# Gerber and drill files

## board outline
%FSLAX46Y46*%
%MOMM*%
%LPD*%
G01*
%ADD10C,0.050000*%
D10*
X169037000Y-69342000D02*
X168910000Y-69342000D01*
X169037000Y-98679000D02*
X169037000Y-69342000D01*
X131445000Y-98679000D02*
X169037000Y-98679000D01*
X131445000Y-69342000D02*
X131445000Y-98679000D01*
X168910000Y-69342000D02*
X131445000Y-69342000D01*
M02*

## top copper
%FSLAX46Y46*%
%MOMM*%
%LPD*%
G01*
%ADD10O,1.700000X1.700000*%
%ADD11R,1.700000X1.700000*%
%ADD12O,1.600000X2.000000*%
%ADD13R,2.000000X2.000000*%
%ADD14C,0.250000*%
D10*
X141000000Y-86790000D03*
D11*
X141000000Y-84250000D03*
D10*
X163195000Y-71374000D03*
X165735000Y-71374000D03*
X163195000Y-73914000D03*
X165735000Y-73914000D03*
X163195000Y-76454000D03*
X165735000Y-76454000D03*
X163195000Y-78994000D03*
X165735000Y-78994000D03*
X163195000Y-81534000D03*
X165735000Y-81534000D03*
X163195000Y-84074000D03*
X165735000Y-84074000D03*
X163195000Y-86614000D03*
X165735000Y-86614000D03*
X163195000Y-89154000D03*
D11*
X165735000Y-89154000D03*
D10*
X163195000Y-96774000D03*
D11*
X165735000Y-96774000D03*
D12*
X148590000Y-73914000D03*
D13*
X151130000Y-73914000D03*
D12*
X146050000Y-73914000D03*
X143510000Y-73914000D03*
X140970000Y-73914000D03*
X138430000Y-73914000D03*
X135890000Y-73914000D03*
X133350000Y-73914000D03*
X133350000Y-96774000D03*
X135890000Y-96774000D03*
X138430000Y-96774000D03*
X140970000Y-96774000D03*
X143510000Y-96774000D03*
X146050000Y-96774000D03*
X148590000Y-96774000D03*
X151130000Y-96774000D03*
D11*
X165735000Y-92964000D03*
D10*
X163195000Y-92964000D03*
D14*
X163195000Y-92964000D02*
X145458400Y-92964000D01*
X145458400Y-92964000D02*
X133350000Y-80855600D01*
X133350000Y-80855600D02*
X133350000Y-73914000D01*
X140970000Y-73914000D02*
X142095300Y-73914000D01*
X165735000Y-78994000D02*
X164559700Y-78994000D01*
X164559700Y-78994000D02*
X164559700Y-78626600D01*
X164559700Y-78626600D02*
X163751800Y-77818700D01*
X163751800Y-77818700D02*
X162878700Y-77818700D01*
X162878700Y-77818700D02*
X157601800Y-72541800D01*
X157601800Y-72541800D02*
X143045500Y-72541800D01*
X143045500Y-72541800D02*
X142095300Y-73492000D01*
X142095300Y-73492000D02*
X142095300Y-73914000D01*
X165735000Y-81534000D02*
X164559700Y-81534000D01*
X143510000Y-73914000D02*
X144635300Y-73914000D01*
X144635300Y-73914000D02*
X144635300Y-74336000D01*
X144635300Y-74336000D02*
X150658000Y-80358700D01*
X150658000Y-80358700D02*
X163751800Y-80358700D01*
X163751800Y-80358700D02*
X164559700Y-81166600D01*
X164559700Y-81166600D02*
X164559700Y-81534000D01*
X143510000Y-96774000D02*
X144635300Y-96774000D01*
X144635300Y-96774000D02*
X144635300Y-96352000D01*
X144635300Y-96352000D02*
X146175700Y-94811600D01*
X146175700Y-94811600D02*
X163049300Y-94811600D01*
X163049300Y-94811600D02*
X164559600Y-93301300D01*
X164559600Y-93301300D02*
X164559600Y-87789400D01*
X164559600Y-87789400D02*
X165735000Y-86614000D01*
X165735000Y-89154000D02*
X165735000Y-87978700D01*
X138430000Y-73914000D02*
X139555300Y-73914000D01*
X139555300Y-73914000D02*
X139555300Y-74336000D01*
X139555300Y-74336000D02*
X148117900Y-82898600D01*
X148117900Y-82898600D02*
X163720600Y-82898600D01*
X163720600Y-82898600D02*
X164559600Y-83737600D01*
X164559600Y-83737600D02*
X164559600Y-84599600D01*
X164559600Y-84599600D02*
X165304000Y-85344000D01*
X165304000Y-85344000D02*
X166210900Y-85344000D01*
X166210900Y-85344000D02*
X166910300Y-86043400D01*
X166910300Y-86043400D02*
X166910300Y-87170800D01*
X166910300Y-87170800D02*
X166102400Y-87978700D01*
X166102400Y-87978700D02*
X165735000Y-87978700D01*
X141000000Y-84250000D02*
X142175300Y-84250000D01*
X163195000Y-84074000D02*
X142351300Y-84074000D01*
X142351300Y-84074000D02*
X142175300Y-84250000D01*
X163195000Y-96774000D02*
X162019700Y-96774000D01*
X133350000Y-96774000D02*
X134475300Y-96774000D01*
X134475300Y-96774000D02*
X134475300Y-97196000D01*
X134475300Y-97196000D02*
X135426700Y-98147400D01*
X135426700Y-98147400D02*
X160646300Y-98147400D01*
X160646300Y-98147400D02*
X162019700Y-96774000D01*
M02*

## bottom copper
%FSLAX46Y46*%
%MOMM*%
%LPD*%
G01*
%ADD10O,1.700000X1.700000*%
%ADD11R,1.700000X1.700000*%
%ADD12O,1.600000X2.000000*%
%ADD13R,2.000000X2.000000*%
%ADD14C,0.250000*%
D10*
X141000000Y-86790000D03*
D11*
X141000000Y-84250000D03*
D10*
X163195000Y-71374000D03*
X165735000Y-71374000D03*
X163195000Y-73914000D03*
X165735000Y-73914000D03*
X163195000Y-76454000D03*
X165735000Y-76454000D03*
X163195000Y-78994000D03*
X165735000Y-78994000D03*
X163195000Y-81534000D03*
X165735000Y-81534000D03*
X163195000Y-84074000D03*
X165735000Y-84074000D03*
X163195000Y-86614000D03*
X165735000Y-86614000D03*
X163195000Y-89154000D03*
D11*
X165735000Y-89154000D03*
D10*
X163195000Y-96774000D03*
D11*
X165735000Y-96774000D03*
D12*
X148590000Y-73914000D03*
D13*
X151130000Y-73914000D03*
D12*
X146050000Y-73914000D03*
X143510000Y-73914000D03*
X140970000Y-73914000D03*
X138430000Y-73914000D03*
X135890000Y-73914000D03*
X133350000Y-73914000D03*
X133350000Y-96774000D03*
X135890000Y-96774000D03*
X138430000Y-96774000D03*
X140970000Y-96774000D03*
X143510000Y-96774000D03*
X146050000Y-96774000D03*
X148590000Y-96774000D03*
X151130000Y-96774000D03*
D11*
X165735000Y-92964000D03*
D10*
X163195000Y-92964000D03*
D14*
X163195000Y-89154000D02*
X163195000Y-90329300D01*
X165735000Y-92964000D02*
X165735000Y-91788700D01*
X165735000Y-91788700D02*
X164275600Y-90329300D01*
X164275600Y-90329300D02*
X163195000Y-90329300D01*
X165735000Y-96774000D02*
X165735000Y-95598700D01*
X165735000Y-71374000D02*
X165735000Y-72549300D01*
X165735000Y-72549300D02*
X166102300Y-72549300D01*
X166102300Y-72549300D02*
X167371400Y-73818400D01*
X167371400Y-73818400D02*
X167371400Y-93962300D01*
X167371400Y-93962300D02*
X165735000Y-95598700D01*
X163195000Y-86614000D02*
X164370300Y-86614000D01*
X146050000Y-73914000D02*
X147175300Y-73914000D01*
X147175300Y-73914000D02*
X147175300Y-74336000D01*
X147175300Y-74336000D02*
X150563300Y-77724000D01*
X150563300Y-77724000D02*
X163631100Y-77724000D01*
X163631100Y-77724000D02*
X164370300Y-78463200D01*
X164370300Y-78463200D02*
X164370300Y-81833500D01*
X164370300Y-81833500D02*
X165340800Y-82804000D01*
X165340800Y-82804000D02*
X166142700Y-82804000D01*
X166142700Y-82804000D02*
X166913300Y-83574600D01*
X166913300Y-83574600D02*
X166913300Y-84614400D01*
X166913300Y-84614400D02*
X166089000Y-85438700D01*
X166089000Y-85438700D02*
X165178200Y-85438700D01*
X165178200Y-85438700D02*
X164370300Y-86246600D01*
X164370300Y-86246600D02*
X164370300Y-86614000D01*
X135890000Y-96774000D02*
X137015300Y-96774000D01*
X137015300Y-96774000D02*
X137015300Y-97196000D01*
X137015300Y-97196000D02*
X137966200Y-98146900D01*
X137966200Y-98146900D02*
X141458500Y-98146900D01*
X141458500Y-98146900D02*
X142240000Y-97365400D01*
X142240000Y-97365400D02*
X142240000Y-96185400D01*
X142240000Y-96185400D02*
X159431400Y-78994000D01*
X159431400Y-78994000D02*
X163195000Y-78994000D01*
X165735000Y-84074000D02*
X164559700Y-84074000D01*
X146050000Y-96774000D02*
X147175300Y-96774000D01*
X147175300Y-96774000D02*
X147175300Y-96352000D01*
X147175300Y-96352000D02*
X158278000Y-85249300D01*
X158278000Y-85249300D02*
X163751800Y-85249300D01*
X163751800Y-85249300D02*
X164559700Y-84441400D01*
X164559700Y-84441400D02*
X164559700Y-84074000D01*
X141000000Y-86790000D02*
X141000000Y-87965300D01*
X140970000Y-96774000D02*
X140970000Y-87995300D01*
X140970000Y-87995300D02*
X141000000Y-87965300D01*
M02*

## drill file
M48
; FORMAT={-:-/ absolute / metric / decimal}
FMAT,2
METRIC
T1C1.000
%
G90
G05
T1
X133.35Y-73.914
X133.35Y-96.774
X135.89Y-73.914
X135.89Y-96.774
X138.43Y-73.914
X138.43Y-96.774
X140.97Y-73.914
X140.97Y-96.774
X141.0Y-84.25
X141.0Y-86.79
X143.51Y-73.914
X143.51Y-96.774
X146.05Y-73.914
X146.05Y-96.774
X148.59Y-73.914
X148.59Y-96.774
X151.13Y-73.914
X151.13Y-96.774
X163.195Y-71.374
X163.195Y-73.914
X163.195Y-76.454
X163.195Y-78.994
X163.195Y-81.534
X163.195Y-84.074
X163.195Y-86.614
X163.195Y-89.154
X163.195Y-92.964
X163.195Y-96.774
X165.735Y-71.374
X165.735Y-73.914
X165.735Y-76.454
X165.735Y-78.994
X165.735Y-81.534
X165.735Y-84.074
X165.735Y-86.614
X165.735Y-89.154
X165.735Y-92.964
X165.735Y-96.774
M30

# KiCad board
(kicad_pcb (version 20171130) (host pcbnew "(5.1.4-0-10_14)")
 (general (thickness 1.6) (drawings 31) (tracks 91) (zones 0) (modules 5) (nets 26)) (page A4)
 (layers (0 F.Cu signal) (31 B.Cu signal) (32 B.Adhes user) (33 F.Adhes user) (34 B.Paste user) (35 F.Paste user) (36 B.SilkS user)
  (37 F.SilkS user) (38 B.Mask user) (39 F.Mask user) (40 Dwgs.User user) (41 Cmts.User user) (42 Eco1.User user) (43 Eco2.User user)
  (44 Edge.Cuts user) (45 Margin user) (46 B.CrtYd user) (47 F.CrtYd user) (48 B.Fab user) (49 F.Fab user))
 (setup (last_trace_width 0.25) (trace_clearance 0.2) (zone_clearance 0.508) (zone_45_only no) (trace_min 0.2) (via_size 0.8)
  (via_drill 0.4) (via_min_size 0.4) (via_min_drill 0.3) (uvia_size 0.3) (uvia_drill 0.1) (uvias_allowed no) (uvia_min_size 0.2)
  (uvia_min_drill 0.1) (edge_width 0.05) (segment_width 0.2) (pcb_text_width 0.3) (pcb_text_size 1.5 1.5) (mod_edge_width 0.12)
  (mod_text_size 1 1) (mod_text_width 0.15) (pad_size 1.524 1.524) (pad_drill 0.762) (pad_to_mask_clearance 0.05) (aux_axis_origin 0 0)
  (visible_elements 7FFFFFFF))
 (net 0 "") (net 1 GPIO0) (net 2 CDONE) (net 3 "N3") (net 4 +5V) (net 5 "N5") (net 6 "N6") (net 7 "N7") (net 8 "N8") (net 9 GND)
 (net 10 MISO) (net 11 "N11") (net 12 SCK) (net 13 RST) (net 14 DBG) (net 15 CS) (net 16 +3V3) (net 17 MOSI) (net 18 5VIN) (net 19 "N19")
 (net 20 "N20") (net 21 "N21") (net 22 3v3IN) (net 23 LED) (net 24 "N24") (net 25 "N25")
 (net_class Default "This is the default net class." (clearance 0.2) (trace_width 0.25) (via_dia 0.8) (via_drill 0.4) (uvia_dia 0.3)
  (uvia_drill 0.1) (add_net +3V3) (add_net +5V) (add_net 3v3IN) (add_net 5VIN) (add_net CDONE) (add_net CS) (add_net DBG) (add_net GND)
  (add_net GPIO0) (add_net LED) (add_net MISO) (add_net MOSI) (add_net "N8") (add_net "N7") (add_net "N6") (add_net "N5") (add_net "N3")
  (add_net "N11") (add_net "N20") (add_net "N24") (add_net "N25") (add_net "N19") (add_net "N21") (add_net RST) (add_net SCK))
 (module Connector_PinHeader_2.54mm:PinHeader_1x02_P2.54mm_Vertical (layer F.Cu) (at 141 84.25)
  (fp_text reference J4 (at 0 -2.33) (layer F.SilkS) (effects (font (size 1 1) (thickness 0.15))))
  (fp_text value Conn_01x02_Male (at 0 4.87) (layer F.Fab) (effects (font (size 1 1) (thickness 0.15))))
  (pad 2 thru_hole oval (at 0 2.54) (size 1.7 1.7) (drill 1) (layers *.Cu *.Mask) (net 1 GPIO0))
  (pad 1 thru_hole rect (at 0 0) (size 1.7 1.7) (drill 1) (layers *.Cu *.Mask) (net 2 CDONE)))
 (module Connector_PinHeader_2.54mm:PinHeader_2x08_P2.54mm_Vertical (layer F.Cu) (at 165.735 89.154 180)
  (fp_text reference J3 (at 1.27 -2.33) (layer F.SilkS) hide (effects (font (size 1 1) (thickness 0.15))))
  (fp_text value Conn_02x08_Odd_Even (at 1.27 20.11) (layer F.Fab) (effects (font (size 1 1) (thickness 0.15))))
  (pad 16 thru_hole oval (at 2.54 17.78 180) (size 1.7 1.7) (drill 1) (layers *.Cu *.Mask) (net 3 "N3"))
  (pad 15 thru_hole oval (at 0 17.78 180) (size 1.7 1.7) (drill 1) (layers *.Cu *.Mask) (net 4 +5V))
  (pad 14 thru_hole oval (at 2.54 15.24 180) (size 1.7 1.7) (drill 1) (layers *.Cu *.Mask) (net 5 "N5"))
  (pad 13 thru_hole oval (at 0 15.24 180) (size 1.7 1.7) (drill 1) (layers *.Cu *.Mask) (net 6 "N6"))
  (pad 12 thru_hole oval (at 2.54 12.7 180) (size 1.7 1.7) (drill 1) (layers *.Cu *.Mask) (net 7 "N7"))
  (pad 11 thru_hole oval (at 0 12.7 180) (size 1.7 1.7) (drill 1) (layers *.Cu *.Mask) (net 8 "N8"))
  (pad 10 thru_hole oval (at 2.54 10.16 180) (size 1.7 1.7) (drill 1) (layers *.Cu *.Mask) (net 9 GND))
  (pad 9 thru_hole oval (at 0 10.16 180) (size 1.7 1.7) (drill 1) (layers *.Cu *.Mask) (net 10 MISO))
  (pad 8 thru_hole oval (at 2.54 7.62 180) (size 1.7 1.7) (drill 1) (layers *.Cu *.Mask) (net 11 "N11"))
  (pad 7 thru_hole oval (at 0 7.62 180) (size 1.7 1.7) (drill 1) (layers *.Cu *.Mask) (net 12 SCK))
  (pad 6 thru_hole oval (at 2.54 5.08 180) (size 1.7 1.7) (drill 1) (layers *.Cu *.Mask) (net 2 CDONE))
  (pad 5 thru_hole oval (at 0 5.08 180) (size 1.7 1.7) (drill 1) (layers *.Cu *.Mask) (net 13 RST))
  (pad 4 thru_hole oval (at 2.54 2.54 180) (size 1.7 1.7) (drill 1) (layers *.Cu *.Mask) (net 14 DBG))
  (pad 3 thru_hole oval (at 0 2.54 180) (size 1.7 1.7) (drill 1) (layers *.Cu *.Mask) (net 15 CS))
  (pad 2 thru_hole oval (at 2.54 0 180) (size 1.7 1.7) (drill 1) (layers *.Cu *.Mask) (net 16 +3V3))
  (pad 1 thru_hole rect (at 0 0 180) (size 1.7 1.7) (drill 1) (layers *.Cu *.Mask) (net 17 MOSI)))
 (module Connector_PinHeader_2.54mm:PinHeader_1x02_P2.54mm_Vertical (layer F.Cu) (at 165.735 96.774 270)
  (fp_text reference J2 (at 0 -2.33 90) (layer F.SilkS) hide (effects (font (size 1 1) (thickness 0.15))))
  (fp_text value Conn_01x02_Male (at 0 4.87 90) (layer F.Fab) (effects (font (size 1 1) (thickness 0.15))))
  (pad 2 thru_hole oval (at 0 2.54 270) (size 1.7 1.7) (drill 1) (layers *.Cu *.Mask) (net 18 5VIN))
  (pad 1 thru_hole rect (at 0 0 270) (size 1.7 1.7) (drill 1) (layers *.Cu *.Mask) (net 4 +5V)))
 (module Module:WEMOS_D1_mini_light (layer F.Cu) (at 151.13 73.914 270)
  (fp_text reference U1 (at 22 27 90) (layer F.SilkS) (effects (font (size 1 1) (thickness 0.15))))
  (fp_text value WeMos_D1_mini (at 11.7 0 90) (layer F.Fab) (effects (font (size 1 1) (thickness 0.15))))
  (pad 2 thru_hole oval (at 0 2.54 270) (size 2 1.6) (drill 1) (layers *.Cu *.Mask) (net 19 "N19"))
  (pad 1 thru_hole rect (at 0 0 270) (size 2 2) (drill 1) (layers *.Cu *.Mask) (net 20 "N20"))
  (pad 3 thru_hole oval (at 0 5.08 270) (size 2 1.6) (drill 1) (layers *.Cu *.Mask) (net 14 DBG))
  (pad 4 thru_hole oval (at 0 7.62 270) (size 2 1.6) (drill 1) (layers *.Cu *.Mask) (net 12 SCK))
  (pad 5 thru_hole oval (at 0 10.16 270) (size 2 1.6) (drill 1) (layers *.Cu *.Mask) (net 10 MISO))
  (pad 6 thru_hole oval (at 0 12.7 270) (size 2 1.6) (drill 1) (layers *.Cu *.Mask) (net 17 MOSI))
  (pad 7 thru_hole oval (at 0 15.24 270) (size 2 1.6) (drill 1) (layers *.Cu *.Mask) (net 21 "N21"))
  (pad 8 thru_hole oval (at 0 17.78 270) (size 2 1.6) (drill 1) (layers *.Cu *.Mask) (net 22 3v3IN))
  (pad 9 thru_hole oval (at 22.86 17.78 270) (size 2 1.6) (drill 1) (layers *.Cu *.Mask) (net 18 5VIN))
  (pad 10 thru_hole oval (at 22.86 15.24 270) (size 2 1.6) (drill 1) (layers *.Cu *.Mask) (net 9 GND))
  (pad 11 thru_hole oval (at 22.86 12.7 270) (size 2 1.6) (drill 1) (layers *.Cu *.Mask) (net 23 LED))
  (pad 12 thru_hole oval (at 22.86 10.16 270) (size 2 1.6) (drill 1) (layers *.Cu *.Mask) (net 1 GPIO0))
  (pad 13 thru_hole oval (at 22.86 7.62 270) (size 2 1.6) (drill 1) (layers *.Cu *.Mask) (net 15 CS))
  (pad 14 thru_hole oval (at 22.86 5.08 270) (size 2 1.6) (drill 1) (layers *.Cu *.Mask) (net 13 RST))
  (pad 15 thru_hole oval (at 22.86 2.54 270) (size 2 1.6) (drill 1) (layers *.Cu *.Mask) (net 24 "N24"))
  (pad 16 thru_hole oval (at 22.86 0 270) (size 2 1.6) (drill 1) (layers *.Cu *.Mask) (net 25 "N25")))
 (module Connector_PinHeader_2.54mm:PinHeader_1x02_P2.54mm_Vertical (layer F.Cu) (at 165.735 92.964 270)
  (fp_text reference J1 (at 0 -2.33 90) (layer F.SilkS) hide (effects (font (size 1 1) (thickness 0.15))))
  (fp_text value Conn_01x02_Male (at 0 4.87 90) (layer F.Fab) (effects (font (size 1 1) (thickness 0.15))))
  (pad 1 thru_hole rect (at 0 0 270) (size 1.7 1.7) (drill 1) (layers *.Cu *.Mask) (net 16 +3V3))
  (pad 2 thru_hole oval (at 0 2.54 270) (size 1.7 1.7) (drill 1) (layers *.Cu *.Mask) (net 22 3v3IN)))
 (gr_line (start 169.037 69.342) (end 168.91 69.342) (layer Edge.Cuts) (width 0.05))
 (gr_line (start 169.037 98.679) (end 169.037 69.342) (layer Edge.Cuts) (width 0.05))
 (gr_line (start 131.445 98.679) (end 169.037 98.679) (layer Edge.Cuts) (width 0.05))
 (gr_line (start 131.445 69.342) (end 131.445 98.679) (layer Edge.Cuts) (width 0.05))
 (gr_line (start 168.91 69.342) (end 131.445 69.342) (layer Edge.Cuts) (width 0.05))
 (segment (start 163.195 92.964) (end 145.4584 92.964) (width 0.25) (layer F.Cu) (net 22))
 (segment (start 145.4584 92.964) (end 133.35 80.8556) (width 0.25) (layer F.Cu) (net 22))
 (segment (start 133.35 80.8556) (end 133.35 73.914) (width 0.25) (layer F.Cu) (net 22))
 (segment (start 163.195 89.154) (end 163.195 90.3293) (width 0.25) (layer B.Cu) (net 16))
 (segment (start 165.735 92.964) (end 165.735 91.7887) (width 0.25) (layer B.Cu) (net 16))
 (segment (start 165.735 91.7887) (end 164.2756 90.3293) (width 0.25) (layer B.Cu) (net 16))
 (segment (start 164.2756 90.3293) (end 163.195 90.3293) (width 0.25) (layer B.Cu) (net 16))
 (segment (start 165.735 96.774) (end 165.735 95.5987) (width 0.25) (layer B.Cu) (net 4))
 (segment (start 165.735 71.374) (end 165.735 72.5493) (width 0.25) (layer B.Cu) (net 4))
 (segment (start 165.735 72.5493) (end 166.1023 72.5493) (width 0.25) (layer B.Cu) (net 4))
 (segment (start 166.1023 72.5493) (end 167.3714 73.8184) (width 0.25) (layer B.Cu) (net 4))
 (segment (start 167.3714 73.8184) (end 167.3714 93.9623) (width 0.25) (layer B.Cu) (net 4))
 (segment (start 167.3714 93.9623) (end 165.735 95.5987) (width 0.25) (layer B.Cu) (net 4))
 (segment (start 163.195 86.614) (end 164.3703 86.614) (width 0.25) (layer B.Cu) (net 14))
 (segment (start 146.05 73.914) (end 147.1753 73.914) (width 0.25) (layer B.Cu) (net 14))
 (segment (start 147.1753 73.914) (end 147.1753 74.336) (width 0.25) (layer B.Cu) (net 14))
 (segment (start 147.1753 74.336) (end 150.5633 77.724) (width 0.25) (layer B.Cu) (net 14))
 (segment (start 150.5633 77.724) (end 163.6311 77.724) (width 0.25) (layer B.Cu) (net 14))
 (segment (start 163.6311 77.724) (end 164.3703 78.4632) (width 0.25) (layer B.Cu) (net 14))
 (segment (start 164.3703 78.4632) (end 164.3703 81.8335) (width 0.25) (layer B.Cu) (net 14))
 (segment (start 164.3703 81.8335) (end 165.3408 82.804) (width 0.25) (layer B.Cu) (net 14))
 (segment (start 165.3408 82.804) (end 166.1427 82.804) (width 0.25) (layer B.Cu) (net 14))
 (segment (start 166.1427 82.804) (end 166.9133 83.5746) (width 0.25) (layer B.Cu) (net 14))
 (segment (start 166.9133 83.5746) (end 166.9133 84.6144) (width 0.25) (layer B.Cu) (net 14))
 (segment (start 166.9133 84.6144) (end 166.089 85.4387) (width 0.25) (layer B.Cu) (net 14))
 (segment (start 166.089 85.4387) (end 165.1782 85.4387) (width 0.25) (layer B.Cu) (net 14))
 (segment (start 165.1782 85.4387) (end 164.3703 86.2466) (width 0.25) (layer B.Cu) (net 14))
 (segment (start 164.3703 86.2466) (end 164.3703 86.614) (width 0.25) (layer B.Cu) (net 14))
 (segment (start 135.89 96.774) (end 137.0153 96.774) (width 0.25) (layer B.Cu) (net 9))
 (segment (start 137.0153 96.774) (end 137.0153 97.196) (width 0.25) (layer B.Cu) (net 9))
 (segment (start 137.0153 97.196) (end 137.9662 98.1469) (width 0.25) (layer B.Cu) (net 9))
 (segment (start 137.9662 98.1469) (end 141.4585 98.1469) (width 0.25) (layer B.Cu) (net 9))
 (segment (start 141.4585 98.1469) (end 142.24 97.3654) (width 0.25) (layer B.Cu) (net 9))
 (segment (start 142.24 97.3654) (end 142.24 96.1854) (width 0.25) (layer B.Cu) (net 9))
 (segment (start 142.24 96.1854) (end 159.4314 78.994) (width 0.25) (layer B.Cu) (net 9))
 (segment (start 159.4314 78.994) (end 163.195 78.994) (width 0.25) (layer B.Cu) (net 9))
 (segment (start 140.97 73.914) (end 142.0953 73.914) (width 0.25) (layer F.Cu) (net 10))
 (segment (start 165.735 78.994) (end 164.5597 78.994) (width 0.25) (layer F.Cu) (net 10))
 (segment (start 164.5597 78.994) (end 164.5597 78.6266) (width 0.25) (layer F.Cu) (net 10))
 (segment (start 164.5597 78.6266) (end 163.7518 77.8187) (width 0.25) (layer F.Cu) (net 10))
 (segment (start 163.7518 77.8187) (end 162.8787 77.8187) (width 0.25) (layer F.Cu) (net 10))
 (segment (start 162.8787 77.8187) (end 157.6018 72.5418) (width 0.25) (layer F.Cu) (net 10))
 (segment (start 157.6018 72.5418) (end 143.0455 72.5418) (width 0.25) (layer F.Cu) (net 10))
 (segment (start 143.0455 72.5418) (end 142.0953 73.492) (width 0.25) (layer F.Cu) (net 10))
 (segment (start 142.0953 73.492) (end 142.0953 73.914) (width 0.25) (layer F.Cu) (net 10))
 (segment (start 165.735 81.534) (end 164.5597 81.534) (width 0.25) (layer F.Cu) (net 12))
 (segment (start 143.51 73.914) (end 144.6353 73.914) (width 0.25) (layer F.Cu) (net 12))
 (segment (start 144.6353 73.914) (end 144.6353 74.336) (width 0.25) (layer F.Cu) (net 12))
 (segment (start 144.6353 74.336) (end 150.658 80.3587) (width 0.25) (layer F.Cu) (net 12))
 (segment (start 150.658 80.3587) (end 163.7518 80.3587) (width 0.25) (layer F.Cu) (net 12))
 (segment (start 163.7518 80.3587) (end 164.5597 81.1666) (width 0.25) (layer F.Cu) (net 12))
 (segment (start 164.5597 81.1666) (end 164.5597 81.534) (width 0.25) (layer F.Cu) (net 12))
 (segment (start 165.735 84.074) (end 164.5597 84.074) (width 0.25) (layer B.Cu) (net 13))
 (segment (start 146.05 96.774) (end 147.1753 96.774) (width 0.25) (layer B.Cu) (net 13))
 (segment (start 147.1753 96.774) (end 147.1753 96.352) (width 0.25) (layer B.Cu) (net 13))
 (segment (start 147.1753 96.352) (end 158.278 85.2493) (width 0.25) (layer B.Cu) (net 13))
 (segment (start 158.278 85.2493) (end 163.7518 85.2493) (width 0.25) (layer B.Cu) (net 13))
 (segment (start 163.7518 85.2493) (end 164.5597 84.4414) (width 0.25) (layer B.Cu) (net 13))
 (segment (start 164.5597 84.4414) (end 164.5597 84.074) (width 0.25) (layer B.Cu) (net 13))
 (segment (start 143.51 96.774) (end 144.6353 96.774) (width 0.25) (layer F.Cu) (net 15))
 (segment (start 144.6353 96.774) (end 144.6353 96.352) (width 0.25) (layer F.Cu) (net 15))
 (segment (start 144.6353 96.352) (end 146.1757 94.8116) (width 0.25) (layer F.Cu) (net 15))
 (segment (start 146.1757 94.8116) (end 163.0493 94.8116) (width 0.25) (layer F.Cu) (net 15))
 (segment (start 163.0493 94.8116) (end 164.5596 93.3013) (width 0.25) (layer F.Cu) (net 15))
 (segment (start 164.5596 93.3013) (end 164.5596 87.7894) (width 0.25) (layer F.Cu) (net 15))
 (segment (start 164.5596 87.7894) (end 165.735 86.614) (width 0.25) (layer F.Cu) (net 15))
 (segment (start 165.735 89.154) (end 165.735 87.9787) (width 0.25) (layer F.Cu) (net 17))
 (segment (start 138.43 73.914) (end 139.5553 73.914) (width 0.25) (layer F.Cu) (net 17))
 (segment (start 139.5553 73.914) (end 139.5553 74.336) (width 0.25) (layer F.Cu) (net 17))
 (segment (start 139.5553 74.336) (end 148.1179 82.8986) (width 0.25) (layer F.Cu) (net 17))
 (segment (start 148.1179 82.8986) (end 163.7206 82.8986) (width 0.25) (layer F.Cu) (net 17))
 (segment (start 163.7206 82.8986) (end 164.5596 83.7376) (width 0.25) (layer F.Cu) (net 17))
 (segment (start 164.5596 83.7376) (end 164.5596 84.5996) (width 0.25) (layer F.Cu) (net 17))
 (segment (start 164.5596 84.5996) (end 165.304 85.344) (width 0.25) (layer F.Cu) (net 17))
 (segment (start 165.304 85.344) (end 166.2109 85.344) (width 0.25) (layer F.Cu) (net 17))
 (segment (start 166.2109 85.344) (end 166.9103 86.0434) (width 0.25) (layer F.Cu) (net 17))
 (segment (start 166.9103 86.0434) (end 166.9103 87.1708) (width 0.25) (layer F.Cu) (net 17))
 (segment (start 166.9103 87.1708) (end 166.1024 87.9787) (width 0.25) (layer F.Cu) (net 17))
 (segment (start 166.1024 87.9787) (end 165.735 87.9787) (width 0.25) (layer F.Cu) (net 17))
 (segment (start 141 84.25) (end 142.1753 84.25) (width 0.25) (layer F.Cu) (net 2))
 (segment (start 163.195 84.074) (end 142.3513 84.074) (width 0.25) (layer F.Cu) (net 2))
 (segment (start 142.3513 84.074) (end 142.1753 84.25) (width 0.25) (layer F.Cu) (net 2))
 (segment (start 163.195 96.774) (end 162.0197 96.774) (width 0.25) (layer F.Cu) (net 18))
 (segment (start 133.35 96.774) (end 134.4753 96.774) (width 0.25) (layer F.Cu) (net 18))
 (segment (start 134.4753 96.774) (end 134.4753 97.196) (width 0.25) (layer F.Cu) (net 18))
 (segment (start 134.4753 97.196) (end 135.4267 98.1474) (width 0.25) (layer F.Cu) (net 18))
 (segment (start 135.4267 98.1474) (end 160.6463 98.1474) (width 0.25) (layer F.Cu) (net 18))
 (segment (start 160.6463 98.1474) (end 162.0197 96.774) (width 0.25) (layer F.Cu) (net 18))
 (segment (start 141 86.79) (end 141 87.9653) (width 0.25) (layer B.Cu) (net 1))
 (segment (start 140.97 96.774) (end 140.97 87.9953) (width 0.25) (layer B.Cu) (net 1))
 (segment (start 140.97 87.9953) (end 141 87.9653) (width 0.25) (layer B.Cu) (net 1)))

